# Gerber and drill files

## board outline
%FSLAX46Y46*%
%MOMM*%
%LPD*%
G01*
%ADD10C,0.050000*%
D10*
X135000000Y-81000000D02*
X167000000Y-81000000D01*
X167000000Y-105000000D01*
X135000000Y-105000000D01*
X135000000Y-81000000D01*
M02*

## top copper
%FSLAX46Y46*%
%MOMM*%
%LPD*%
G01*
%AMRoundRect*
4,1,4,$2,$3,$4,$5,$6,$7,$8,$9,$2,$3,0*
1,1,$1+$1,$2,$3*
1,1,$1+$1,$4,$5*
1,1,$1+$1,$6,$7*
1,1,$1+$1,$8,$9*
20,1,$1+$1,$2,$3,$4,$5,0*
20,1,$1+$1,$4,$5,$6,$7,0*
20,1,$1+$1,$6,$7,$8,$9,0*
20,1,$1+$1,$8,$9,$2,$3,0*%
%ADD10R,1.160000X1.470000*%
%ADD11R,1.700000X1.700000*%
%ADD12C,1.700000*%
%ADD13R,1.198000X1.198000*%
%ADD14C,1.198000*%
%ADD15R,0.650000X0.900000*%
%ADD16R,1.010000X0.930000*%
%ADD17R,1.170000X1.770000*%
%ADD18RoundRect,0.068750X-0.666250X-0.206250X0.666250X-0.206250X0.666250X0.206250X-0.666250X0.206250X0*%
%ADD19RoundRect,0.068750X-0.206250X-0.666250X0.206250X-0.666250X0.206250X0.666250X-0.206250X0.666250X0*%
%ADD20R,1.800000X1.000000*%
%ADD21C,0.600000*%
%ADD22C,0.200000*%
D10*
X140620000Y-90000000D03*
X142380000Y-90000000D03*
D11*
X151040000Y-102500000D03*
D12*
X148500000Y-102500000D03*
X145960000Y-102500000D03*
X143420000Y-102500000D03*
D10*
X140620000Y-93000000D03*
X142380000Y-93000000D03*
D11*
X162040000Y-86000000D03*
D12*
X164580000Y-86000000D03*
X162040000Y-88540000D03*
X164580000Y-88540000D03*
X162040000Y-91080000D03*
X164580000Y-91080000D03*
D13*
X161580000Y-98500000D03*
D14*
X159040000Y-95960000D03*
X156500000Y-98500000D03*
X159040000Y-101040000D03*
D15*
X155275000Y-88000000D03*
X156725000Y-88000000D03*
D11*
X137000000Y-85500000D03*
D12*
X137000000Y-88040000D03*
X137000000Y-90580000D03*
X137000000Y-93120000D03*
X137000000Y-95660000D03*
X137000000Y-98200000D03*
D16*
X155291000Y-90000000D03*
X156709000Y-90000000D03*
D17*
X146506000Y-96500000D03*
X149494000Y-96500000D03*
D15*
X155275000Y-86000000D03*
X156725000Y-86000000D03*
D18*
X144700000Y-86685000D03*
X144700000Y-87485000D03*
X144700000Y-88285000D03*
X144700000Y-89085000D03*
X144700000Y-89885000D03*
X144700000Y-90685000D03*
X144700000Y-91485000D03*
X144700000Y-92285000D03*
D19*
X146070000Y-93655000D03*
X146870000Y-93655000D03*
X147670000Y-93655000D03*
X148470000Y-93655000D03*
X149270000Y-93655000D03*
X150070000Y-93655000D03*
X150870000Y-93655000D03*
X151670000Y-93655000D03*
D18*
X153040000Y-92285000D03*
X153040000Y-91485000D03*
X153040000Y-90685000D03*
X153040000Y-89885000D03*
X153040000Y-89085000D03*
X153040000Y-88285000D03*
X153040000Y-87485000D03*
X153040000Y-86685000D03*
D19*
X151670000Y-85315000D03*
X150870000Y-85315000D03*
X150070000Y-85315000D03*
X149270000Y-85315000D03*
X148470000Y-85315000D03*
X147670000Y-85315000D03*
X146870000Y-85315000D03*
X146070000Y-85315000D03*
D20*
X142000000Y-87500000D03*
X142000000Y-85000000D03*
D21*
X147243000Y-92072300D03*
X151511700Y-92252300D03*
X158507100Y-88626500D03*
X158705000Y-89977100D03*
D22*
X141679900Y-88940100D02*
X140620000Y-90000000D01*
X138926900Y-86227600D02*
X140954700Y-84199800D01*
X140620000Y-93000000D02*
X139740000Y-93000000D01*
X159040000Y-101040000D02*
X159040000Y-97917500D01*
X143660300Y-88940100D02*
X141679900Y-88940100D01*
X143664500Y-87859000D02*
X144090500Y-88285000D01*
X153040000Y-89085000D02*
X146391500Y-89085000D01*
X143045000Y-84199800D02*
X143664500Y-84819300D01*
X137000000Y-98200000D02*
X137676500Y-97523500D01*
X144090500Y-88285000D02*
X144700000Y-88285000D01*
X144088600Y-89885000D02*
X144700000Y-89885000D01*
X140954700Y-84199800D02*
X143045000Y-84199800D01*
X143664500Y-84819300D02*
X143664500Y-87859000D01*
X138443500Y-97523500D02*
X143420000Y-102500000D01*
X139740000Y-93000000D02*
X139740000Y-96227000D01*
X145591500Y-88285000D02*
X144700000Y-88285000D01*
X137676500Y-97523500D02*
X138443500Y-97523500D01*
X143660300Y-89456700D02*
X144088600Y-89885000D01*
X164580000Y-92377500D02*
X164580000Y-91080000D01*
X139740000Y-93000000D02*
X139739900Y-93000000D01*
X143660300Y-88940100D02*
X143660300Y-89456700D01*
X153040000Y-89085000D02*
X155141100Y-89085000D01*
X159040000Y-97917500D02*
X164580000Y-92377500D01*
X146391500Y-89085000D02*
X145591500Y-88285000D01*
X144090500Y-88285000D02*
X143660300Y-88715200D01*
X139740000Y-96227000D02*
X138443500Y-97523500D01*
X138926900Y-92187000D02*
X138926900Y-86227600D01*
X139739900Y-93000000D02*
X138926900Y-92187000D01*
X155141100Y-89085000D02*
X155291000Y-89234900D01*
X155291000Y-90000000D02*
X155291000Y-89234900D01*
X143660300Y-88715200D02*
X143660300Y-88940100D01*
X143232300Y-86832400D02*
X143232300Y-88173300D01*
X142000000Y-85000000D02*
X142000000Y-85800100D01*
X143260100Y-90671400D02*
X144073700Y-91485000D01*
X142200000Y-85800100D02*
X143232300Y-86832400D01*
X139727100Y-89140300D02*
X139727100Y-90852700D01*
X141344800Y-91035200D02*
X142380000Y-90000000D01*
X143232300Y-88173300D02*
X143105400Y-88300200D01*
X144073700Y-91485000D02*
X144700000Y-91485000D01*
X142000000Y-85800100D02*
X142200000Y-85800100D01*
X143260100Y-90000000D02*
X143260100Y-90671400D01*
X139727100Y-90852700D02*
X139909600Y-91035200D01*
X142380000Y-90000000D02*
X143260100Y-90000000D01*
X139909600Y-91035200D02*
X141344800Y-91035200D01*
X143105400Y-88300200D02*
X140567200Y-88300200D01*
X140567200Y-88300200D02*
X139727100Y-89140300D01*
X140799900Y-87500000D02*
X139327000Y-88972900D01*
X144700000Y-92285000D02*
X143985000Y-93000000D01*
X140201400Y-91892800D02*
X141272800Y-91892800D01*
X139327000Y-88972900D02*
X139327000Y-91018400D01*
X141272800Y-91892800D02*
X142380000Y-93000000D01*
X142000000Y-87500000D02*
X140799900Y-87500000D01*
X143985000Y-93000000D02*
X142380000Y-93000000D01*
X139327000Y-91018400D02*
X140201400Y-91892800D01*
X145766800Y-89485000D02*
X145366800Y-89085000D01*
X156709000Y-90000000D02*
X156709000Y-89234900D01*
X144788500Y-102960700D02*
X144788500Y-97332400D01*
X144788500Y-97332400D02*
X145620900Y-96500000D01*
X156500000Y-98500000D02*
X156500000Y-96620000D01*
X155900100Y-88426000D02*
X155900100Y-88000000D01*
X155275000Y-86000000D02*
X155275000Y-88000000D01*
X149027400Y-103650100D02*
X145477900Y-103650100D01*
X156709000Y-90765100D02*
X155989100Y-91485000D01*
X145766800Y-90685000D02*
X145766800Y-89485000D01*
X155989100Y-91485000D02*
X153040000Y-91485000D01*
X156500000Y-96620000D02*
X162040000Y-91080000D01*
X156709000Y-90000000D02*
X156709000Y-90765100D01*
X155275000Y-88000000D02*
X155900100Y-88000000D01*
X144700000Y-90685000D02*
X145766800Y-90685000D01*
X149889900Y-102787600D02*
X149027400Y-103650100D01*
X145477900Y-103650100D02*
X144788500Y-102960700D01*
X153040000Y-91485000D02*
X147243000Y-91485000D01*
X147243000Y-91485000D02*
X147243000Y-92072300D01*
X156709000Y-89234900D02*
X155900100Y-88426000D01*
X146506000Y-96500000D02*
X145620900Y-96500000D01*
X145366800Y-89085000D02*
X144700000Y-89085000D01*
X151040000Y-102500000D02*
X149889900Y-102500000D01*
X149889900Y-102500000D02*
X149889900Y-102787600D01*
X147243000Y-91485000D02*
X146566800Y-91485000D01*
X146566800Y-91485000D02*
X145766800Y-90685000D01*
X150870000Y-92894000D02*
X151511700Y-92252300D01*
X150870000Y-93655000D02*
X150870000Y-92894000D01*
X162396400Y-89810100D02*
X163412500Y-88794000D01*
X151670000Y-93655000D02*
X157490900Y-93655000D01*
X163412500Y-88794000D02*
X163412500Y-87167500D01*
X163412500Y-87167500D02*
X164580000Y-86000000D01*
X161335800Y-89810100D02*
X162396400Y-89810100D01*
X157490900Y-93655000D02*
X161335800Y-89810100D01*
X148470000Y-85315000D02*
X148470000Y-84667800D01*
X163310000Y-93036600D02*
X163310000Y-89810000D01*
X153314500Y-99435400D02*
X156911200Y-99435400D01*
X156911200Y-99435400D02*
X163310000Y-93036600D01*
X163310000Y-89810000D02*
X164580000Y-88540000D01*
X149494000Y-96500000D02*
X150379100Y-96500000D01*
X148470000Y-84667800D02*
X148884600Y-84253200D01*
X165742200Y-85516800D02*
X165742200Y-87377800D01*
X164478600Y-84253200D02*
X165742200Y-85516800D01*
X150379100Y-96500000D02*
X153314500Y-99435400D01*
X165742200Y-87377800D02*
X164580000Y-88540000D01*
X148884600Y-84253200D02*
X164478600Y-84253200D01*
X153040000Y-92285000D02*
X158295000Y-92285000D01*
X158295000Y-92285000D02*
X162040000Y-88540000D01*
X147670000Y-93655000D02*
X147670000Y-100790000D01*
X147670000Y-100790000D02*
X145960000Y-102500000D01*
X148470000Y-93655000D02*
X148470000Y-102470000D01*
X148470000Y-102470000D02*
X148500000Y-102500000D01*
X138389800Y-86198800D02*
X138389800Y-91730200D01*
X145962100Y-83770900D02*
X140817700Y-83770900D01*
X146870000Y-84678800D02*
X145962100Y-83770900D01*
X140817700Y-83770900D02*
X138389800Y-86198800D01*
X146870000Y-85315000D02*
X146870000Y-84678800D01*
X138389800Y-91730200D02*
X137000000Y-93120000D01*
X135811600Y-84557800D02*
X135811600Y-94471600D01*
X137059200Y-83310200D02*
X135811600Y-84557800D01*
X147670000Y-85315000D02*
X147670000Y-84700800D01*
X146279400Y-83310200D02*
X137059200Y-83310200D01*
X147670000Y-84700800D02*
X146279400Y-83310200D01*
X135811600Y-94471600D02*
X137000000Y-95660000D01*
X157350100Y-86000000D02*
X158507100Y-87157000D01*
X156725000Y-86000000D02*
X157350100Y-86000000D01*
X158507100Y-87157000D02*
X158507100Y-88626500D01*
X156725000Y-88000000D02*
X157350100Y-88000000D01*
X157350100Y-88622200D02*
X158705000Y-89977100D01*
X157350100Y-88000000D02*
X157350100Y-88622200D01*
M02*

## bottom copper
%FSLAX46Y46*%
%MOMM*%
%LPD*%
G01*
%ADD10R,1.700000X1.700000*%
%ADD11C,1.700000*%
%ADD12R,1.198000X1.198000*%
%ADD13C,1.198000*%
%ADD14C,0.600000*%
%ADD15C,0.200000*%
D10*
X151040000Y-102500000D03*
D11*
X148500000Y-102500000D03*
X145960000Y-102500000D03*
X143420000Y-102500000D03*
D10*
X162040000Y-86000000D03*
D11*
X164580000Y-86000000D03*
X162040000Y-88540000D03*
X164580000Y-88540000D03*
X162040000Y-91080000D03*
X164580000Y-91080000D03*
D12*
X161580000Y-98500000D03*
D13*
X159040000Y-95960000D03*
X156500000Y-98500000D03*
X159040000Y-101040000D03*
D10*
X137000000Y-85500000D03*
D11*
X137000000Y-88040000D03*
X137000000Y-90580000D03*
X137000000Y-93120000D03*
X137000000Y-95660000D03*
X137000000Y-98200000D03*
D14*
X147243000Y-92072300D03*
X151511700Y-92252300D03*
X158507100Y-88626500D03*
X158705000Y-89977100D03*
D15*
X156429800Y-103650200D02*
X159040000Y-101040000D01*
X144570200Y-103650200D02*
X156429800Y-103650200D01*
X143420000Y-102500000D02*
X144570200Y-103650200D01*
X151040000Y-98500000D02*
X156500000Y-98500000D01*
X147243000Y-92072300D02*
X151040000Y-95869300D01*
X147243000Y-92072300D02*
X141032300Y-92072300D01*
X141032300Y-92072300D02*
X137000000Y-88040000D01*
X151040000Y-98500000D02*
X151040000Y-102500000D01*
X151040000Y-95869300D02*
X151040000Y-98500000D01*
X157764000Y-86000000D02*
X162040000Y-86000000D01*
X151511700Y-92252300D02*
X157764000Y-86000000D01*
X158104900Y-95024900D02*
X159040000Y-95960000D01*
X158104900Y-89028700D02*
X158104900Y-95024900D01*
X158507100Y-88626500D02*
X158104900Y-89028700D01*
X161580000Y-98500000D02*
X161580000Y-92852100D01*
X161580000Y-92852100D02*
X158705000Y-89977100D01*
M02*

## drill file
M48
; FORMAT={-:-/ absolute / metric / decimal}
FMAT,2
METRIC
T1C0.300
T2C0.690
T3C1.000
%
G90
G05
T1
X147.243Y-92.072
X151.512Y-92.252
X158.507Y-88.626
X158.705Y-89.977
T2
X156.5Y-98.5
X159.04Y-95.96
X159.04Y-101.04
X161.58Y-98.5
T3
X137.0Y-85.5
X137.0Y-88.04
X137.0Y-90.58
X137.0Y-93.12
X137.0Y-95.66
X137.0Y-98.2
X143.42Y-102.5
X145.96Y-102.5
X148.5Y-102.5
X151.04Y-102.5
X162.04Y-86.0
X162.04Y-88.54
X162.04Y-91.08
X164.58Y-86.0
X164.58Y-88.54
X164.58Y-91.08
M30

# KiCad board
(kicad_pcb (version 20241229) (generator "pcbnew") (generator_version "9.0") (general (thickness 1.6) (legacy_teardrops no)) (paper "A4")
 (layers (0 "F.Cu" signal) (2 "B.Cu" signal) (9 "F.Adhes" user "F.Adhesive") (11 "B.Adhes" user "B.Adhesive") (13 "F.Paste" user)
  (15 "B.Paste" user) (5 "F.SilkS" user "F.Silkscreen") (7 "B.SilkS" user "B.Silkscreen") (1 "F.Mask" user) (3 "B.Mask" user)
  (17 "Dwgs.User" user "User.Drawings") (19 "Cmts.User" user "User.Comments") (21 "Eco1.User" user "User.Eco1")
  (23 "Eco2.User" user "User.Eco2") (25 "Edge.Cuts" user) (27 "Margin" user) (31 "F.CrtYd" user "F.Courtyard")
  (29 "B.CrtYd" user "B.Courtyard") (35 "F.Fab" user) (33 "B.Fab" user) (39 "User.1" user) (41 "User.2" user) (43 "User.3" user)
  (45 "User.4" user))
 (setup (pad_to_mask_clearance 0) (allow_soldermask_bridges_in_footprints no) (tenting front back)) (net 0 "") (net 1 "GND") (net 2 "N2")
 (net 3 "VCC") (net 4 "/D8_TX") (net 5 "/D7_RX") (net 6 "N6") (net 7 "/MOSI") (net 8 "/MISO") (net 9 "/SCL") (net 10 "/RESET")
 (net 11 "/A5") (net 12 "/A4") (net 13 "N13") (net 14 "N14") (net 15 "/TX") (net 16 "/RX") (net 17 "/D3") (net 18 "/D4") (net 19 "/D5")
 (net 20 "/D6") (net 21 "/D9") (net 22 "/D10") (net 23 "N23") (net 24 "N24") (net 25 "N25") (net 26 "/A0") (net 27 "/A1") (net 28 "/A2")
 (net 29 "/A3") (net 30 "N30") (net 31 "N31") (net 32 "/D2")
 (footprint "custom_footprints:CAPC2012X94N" (layer "F.Cu") (at 141.5 90)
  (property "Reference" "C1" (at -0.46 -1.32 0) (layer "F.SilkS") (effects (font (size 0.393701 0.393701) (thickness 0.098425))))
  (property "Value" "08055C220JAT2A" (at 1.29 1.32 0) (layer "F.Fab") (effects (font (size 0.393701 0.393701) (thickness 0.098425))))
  (pad "1" smd rect (at -0.88 0) (size 1.16 1.47) (layers "F.Cu" "F.Mask" "F.Paste") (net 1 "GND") (solder_mask_margin 0.102))
  (pad "2" smd rect (at 0.88 0) (size 1.16 1.47) (layers "F.Cu" "F.Mask" "F.Paste") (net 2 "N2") (solder_mask_margin 0.102)))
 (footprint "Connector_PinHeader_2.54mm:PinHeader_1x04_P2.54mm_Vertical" (layer "F.Cu") (at 151.04 102.5 -90)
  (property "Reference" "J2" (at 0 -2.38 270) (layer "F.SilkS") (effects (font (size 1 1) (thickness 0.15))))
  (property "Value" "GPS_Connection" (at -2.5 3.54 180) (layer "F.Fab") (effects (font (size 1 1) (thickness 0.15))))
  (pad "1" thru_hole rect (at 0 0 270) (size 1.7 1.7) (drill 1) (layers "*.Cu" "*.Mask") (remove_unused_layers no) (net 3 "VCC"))
  (pad "2" thru_hole circle (at 0 2.54 270) (size 1.7 1.7) (drill 1) (layers "*.Cu" "*.Mask") (remove_unused_layers no) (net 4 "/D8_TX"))
  (pad "3" thru_hole circle (at 0 5.08 270) (size 1.7 1.7) (drill 1) (layers "*.Cu" "*.Mask") (remove_unused_layers no) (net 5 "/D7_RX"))
  (pad "4" thru_hole circle (at 0 7.62 270) (size 1.7 1.7) (drill 1) (layers "*.Cu" "*.Mask") (remove_unused_layers no) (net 1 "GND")))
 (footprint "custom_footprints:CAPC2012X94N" (layer "F.Cu") (at 141.5 93)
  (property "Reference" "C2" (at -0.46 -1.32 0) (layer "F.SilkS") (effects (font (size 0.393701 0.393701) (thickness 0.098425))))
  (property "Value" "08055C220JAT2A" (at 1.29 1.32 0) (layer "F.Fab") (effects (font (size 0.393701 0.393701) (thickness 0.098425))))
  (pad "1" smd rect (at -0.88 0) (size 1.16 1.47) (layers "F.Cu" "F.Mask" "F.Paste") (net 1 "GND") (solder_mask_margin 0.102))
  (pad "2" smd rect (at 0.88 0) (size 1.16 1.47) (layers "F.Cu" "F.Mask" "F.Paste") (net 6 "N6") (solder_mask_margin 0.102)))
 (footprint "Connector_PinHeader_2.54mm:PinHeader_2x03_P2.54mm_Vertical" (layer "F.Cu") (at 162.04 86)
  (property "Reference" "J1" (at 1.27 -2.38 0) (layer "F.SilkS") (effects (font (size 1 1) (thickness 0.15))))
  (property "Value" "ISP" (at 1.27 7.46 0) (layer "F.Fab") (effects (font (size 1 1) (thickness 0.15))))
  (pad "1" thru_hole rect (at 0 0) (size 1.7 1.7) (drill 1) (layers "*.Cu" "*.Mask") (remove_unused_layers no) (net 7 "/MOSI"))
  (pad "2" thru_hole circle (at 2.54 0) (size 1.7 1.7) (drill 1) (layers "*.Cu" "*.Mask") (remove_unused_layers no) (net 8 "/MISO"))
  (pad "3" thru_hole circle (at 0 2.54) (size 1.7 1.7) (drill 1) (layers "*.Cu" "*.Mask") (remove_unused_layers no) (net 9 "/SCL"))
  (pad "4" thru_hole circle (at 2.54 2.54) (size 1.7 1.7) (drill 1) (layers "*.Cu" "*.Mask") (remove_unused_layers no) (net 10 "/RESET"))
  (pad "5" thru_hole circle (at 0 5.08) (size 1.7 1.7) (drill 1) (layers "*.Cu" "*.Mask") (remove_unused_layers no) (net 3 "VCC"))
  (pad "6" thru_hole circle (at 2.54 5.08) (size 1.7 1.7) (drill 1) (layers "*.Cu" "*.Mask") (remove_unused_layers no) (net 1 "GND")))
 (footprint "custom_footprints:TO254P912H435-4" (layer "F.Cu") (at 159.04 98.5 180)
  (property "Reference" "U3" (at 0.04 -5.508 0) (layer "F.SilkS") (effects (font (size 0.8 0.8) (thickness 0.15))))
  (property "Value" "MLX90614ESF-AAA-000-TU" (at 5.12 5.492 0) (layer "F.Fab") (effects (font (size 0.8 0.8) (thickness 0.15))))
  (pad "1" thru_hole rect (at -2.54 0 180) (size 1.198 1.198) (drill 0.69) (layers "*.Cu" "*.Mask") (remove_unused_layers no) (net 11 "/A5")
   (solder_mask_margin 0.102))
  (pad "2" thru_hole circle (at 0 2.54 180) (size 1.198 1.198) (drill 0.69) (layers "*.Cu" "*.Mask") (remove_unused_layers no)
   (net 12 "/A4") (solder_mask_margin 0.102))
  (pad "3" thru_hole circle (at 2.54 0 180) (size 1.198 1.198) (drill 0.69) (layers "*.Cu" "*.Mask") (remove_unused_layers no) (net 3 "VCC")
   (solder_mask_margin 0.102))
  (pad "4" thru_hole circle (at 0 -2.54 180) (size 1.198 1.198) (drill 0.69) (layers "*.Cu" "*.Mask") (remove_unused_layers no)
   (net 1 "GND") (solder_mask_margin 0.102)))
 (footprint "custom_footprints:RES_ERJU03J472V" (layer "F.Cu") (at 156 88)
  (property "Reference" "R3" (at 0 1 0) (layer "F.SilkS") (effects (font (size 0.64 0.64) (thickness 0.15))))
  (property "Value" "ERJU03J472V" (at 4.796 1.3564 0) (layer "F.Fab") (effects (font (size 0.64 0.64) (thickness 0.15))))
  (pad "1" smd rect (at -0.725 0) (size 0.65 0.9) (layers "F.Cu" "F.Mask" "F.Paste") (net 3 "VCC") (solder_mask_margin 0.102))
  (pad "2" smd rect (at 0.725 0) (size 0.65 0.9) (layers "F.Cu" "F.Mask" "F.Paste") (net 11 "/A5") (solder_mask_margin 0.102)))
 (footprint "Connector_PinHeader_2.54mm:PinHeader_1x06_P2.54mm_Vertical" (layer "F.Cu") (at 137 85.5)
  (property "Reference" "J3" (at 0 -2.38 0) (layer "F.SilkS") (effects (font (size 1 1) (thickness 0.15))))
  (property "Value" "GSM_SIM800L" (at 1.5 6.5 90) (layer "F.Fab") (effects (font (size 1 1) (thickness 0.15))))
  (pad "1" thru_hole rect (at 0 0) (size 1.7 1.7) (drill 1) (layers "*.Cu" "*.Mask") (remove_unused_layers no) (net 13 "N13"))
  (pad "2" thru_hole circle (at 0 2.54) (size 1.7 1.7) (drill 1) (layers "*.Cu" "*.Mask") (remove_unused_layers no) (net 3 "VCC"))
  (pad "3" thru_hole circle (at 0 5.08) (size 1.7 1.7) (drill 1) (layers "*.Cu" "*.Mask") (remove_unused_layers no) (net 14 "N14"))
  (pad "4" thru_hole circle (at 0 7.62) (size 1.7 1.7) (drill 1) (layers "*.Cu" "*.Mask") (remove_unused_layers no) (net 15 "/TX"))
  (pad "5" thru_hole circle (at 0 10.16) (size 1.7 1.7) (drill 1) (layers "*.Cu" "*.Mask") (remove_unused_layers no) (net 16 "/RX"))
  (pad "6" thru_hole circle (at 0 12.7) (size 1.7 1.7) (drill 1) (layers "*.Cu" "*.Mask") (remove_unused_layers no) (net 1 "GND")))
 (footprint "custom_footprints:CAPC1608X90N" (layer "F.Cu") (at 156 90)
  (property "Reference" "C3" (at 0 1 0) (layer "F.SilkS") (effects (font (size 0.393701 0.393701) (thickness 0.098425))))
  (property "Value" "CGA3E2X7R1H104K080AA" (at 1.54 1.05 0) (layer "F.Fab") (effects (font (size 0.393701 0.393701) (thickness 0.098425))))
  (pad "1" smd rect (at -0.709 0) (size 1.01 0.93) (layers "F.Cu" "F.Mask" "F.Paste") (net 1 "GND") (solder_mask_margin 0.102))
  (pad "2" smd rect (at 0.709 0) (size 1.01 0.93) (layers "F.Cu" "F.Mask" "F.Paste") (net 3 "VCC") (solder_mask_margin 0.102)))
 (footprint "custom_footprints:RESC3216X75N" (layer "F.Cu") (at 148 96.5)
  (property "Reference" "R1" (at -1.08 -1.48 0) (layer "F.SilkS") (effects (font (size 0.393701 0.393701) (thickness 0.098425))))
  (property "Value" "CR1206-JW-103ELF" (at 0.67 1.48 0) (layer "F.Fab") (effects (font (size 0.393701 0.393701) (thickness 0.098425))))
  (pad "1" smd rect (at -1.494 0) (size 1.17 1.77) (layers "F.Cu" "F.Mask" "F.Paste") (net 3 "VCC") (solder_mask_margin 0.102))
  (pad "2" smd rect (at 1.494 0) (size 1.17 1.77) (layers "F.Cu" "F.Mask" "F.Paste") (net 10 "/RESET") (solder_mask_margin 0.102)))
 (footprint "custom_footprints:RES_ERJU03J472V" (layer "F.Cu") (at 156 86)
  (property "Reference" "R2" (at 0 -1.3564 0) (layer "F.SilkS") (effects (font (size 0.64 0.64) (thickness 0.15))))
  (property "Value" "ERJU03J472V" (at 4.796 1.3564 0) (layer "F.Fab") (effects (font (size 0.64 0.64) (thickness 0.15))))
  (pad "1" smd rect (at -0.725 0) (size 0.65 0.9) (layers "F.Cu" "F.Mask" "F.Paste") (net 3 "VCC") (solder_mask_margin 0.102))
  (pad "2" smd rect (at 0.725 0) (size 0.65 0.9) (layers "F.Cu" "F.Mask" "F.Paste") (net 12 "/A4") (solder_mask_margin 0.102)))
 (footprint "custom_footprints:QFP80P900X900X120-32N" (layer "F.Cu") (at 148.87 89.485)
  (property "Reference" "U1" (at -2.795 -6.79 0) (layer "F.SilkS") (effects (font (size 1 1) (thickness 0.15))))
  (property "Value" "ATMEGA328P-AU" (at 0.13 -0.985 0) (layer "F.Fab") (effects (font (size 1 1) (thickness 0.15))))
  (pad "1" smd roundrect (at -4.17 -2.8) (size 1.47 0.55) (layers "F.Cu" "F.Mask" "F.Paste") (roundrect_rratio 0.125) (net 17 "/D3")
   (solder_mask_margin 0.102))
  (pad "2" smd roundrect (at -4.17 -2) (size 1.47 0.55) (layers "F.Cu" "F.Mask" "F.Paste") (roundrect_rratio 0.125) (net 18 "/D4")
   (solder_mask_margin 0.102))
  (pad "3" smd roundrect (at -4.17 -1.2) (size 1.47 0.55) (layers "F.Cu" "F.Mask" "F.Paste") (roundrect_rratio 0.125) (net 1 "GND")
   (solder_mask_margin 0.102))
  (pad "4" smd roundrect (at -4.17 -0.4) (size 1.47 0.55) (layers "F.Cu" "F.Mask" "F.Paste") (roundrect_rratio 0.125) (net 3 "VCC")
   (solder_mask_margin 0.102))
  (pad "5" smd roundrect (at -4.17 0.4) (size 1.47 0.55) (layers "F.Cu" "F.Mask" "F.Paste") (roundrect_rratio 0.125) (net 1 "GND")
   (solder_mask_margin 0.102))
  (pad "6" smd roundrect (at -4.17 1.2) (size 1.47 0.55) (layers "F.Cu" "F.Mask" "F.Paste") (roundrect_rratio 0.125) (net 3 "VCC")
   (solder_mask_margin 0.102))
  (pad "7" smd roundrect (at -4.17 2) (size 1.47 0.55) (layers "F.Cu" "F.Mask" "F.Paste") (roundrect_rratio 0.125) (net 2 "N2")
   (solder_mask_margin 0.102))
  (pad "8" smd roundrect (at -4.17 2.8) (size 1.47 0.55) (layers "F.Cu" "F.Mask" "F.Paste") (roundrect_rratio 0.125) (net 6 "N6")
   (solder_mask_margin 0.102))
  (pad "9" smd roundrect (at -2.8 4.17) (size 0.55 1.47) (layers "F.Cu" "F.Mask" "F.Paste") (roundrect_rratio 0.125) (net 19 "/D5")
   (solder_mask_margin 0.102))
  (pad "10" smd roundrect (at -2 4.17) (size 0.55 1.47) (layers "F.Cu" "F.Mask" "F.Paste") (roundrect_rratio 0.125) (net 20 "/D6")
   (solder_mask_margin 0.102))
  (pad "11" smd roundrect (at -1.2 4.17) (size 0.55 1.47) (layers "F.Cu" "F.Mask" "F.Paste") (roundrect_rratio 0.125) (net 5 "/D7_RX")
   (solder_mask_margin 0.102))
  (pad "12" smd roundrect (at -0.4 4.17) (size 0.55 1.47) (layers "F.Cu" "F.Mask" "F.Paste") (roundrect_rratio 0.125) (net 4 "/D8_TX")
   (solder_mask_margin 0.102))
  (pad "13" smd roundrect (at 0.4 4.17) (size 0.55 1.47) (layers "F.Cu" "F.Mask" "F.Paste") (roundrect_rratio 0.125) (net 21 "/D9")
   (solder_mask_margin 0.102))
  (pad "14" smd roundrect (at 1.2 4.17) (size 0.55 1.47) (layers "F.Cu" "F.Mask" "F.Paste") (roundrect_rratio 0.125) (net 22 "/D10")
   (solder_mask_margin 0.102))
  (pad "15" smd roundrect (at 2 4.17) (size 0.55 1.47) (layers "F.Cu" "F.Mask" "F.Paste") (roundrect_rratio 0.125) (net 7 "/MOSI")
   (solder_mask_margin 0.102))
  (pad "16" smd roundrect (at 2.8 4.17) (size 0.55 1.47) (layers "F.Cu" "F.Mask" "F.Paste") (roundrect_rratio 0.125) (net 8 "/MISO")
   (solder_mask_margin 0.102))
  (pad "17" smd roundrect (at 4.17 2.8) (size 1.47 0.55) (layers "F.Cu" "F.Mask" "F.Paste") (roundrect_rratio 0.125) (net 9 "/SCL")
   (solder_mask_margin 0.102))
  (pad "18" smd roundrect (at 4.17 2) (size 1.47 0.55) (layers "F.Cu" "F.Mask" "F.Paste") (roundrect_rratio 0.125) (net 3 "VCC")
   (solder_mask_margin 0.102))
  (pad "19" smd roundrect (at 4.17 1.2) (size 1.47 0.55) (layers "F.Cu" "F.Mask" "F.Paste") (roundrect_rratio 0.125) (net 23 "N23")
   (solder_mask_margin 0.102))
  (pad "20" smd roundrect (at 4.17 0.4) (size 1.47 0.55) (layers "F.Cu" "F.Mask" "F.Paste") (roundrect_rratio 0.125) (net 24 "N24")
   (solder_mask_margin 0.102))
  (pad "21" smd roundrect (at 4.17 -0.4) (size 1.47 0.55) (layers "F.Cu" "F.Mask" "F.Paste") (roundrect_rratio 0.125) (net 1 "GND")
   (solder_mask_margin 0.102))
  (pad "22" smd roundrect (at 4.17 -1.2) (size 1.47 0.55) (layers "F.Cu" "F.Mask" "F.Paste") (roundrect_rratio 0.125) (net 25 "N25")
   (solder_mask_margin 0.102))
  (pad "23" smd roundrect (at 4.17 -2) (size 1.47 0.55) (layers "F.Cu" "F.Mask" "F.Paste") (roundrect_rratio 0.125) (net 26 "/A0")
   (solder_mask_margin 0.102))
  (pad "24" smd roundrect (at 4.17 -2.8) (size 1.47 0.55) (layers "F.Cu" "F.Mask" "F.Paste") (roundrect_rratio 0.125) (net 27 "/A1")
   (solder_mask_margin 0.102))
  (pad "25" smd roundrect (at 2.8 -4.17) (size 0.55 1.47) (layers "F.Cu" "F.Mask" "F.Paste") (roundrect_rratio 0.125) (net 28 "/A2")
   (solder_mask_margin 0.102))
  (pad "26" smd roundrect (at 2 -4.17) (size 0.55 1.47) (layers "F.Cu" "F.Mask" "F.Paste") (roundrect_rratio 0.125) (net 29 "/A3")
   (solder_mask_margin 0.102))
  (pad "27" smd roundrect (at 1.2 -4.17) (size 0.55 1.47) (layers "F.Cu" "F.Mask" "F.Paste") (roundrect_rratio 0.125) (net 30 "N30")
   (solder_mask_margin 0.102))
  (pad "28" smd roundrect (at 0.4 -4.17) (size 0.55 1.47) (layers "F.Cu" "F.Mask" "F.Paste") (roundrect_rratio 0.125) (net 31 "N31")
   (solder_mask_margin 0.102))
  (pad "29" smd roundrect (at -0.4 -4.17) (size 0.55 1.47) (layers "F.Cu" "F.Mask" "F.Paste") (roundrect_rratio 0.125) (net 10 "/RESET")
   (solder_mask_margin 0.102))
  (pad "30" smd roundrect (at -1.2 -4.17) (size 0.55 1.47) (layers "F.Cu" "F.Mask" "F.Paste") (roundrect_rratio 0.125) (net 16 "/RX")
   (solder_mask_margin 0.102))
  (pad "31" smd roundrect (at -2 -4.17) (size 0.55 1.47) (layers "F.Cu" "F.Mask" "F.Paste") (roundrect_rratio 0.125) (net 15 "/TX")
   (solder_mask_margin 0.102))
  (pad "32" smd roundrect (at -2.8 -4.17) (size 0.55 1.47) (layers "F.Cu" "F.Mask" "F.Paste") (roundrect_rratio 0.125) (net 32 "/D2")
   (solder_mask_margin 0.102)))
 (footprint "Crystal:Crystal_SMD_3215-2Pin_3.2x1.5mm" (layer "F.Cu") (at 142 86.25 -90)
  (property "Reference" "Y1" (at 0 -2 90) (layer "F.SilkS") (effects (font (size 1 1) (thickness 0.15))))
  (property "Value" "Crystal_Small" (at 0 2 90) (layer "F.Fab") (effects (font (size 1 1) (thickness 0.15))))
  (pad "1" smd rect (at 1.25 0 270) (size 1 1.8) (layers "F.Cu" "F.Mask" "F.Paste") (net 6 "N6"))
  (pad "2" smd rect (at -1.25 0 270) (size 1 1.8) (layers "F.Cu" "F.Mask" "F.Paste") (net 2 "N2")))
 (gr_rect (start 135 81) (end 167 105) (stroke (width 0.05) (type default)) (fill no) (layer "Edge.Cuts"))
 (segment (start 141.6799 88.9401) (end 140.62 90) (width 0.2) (layer "F.Cu") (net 1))
 (segment (start 138.9269 86.2276) (end 140.9547 84.1998) (width 0.2) (layer "F.Cu") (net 1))
 (segment (start 140.62 93) (end 139.74 93) (width 0.2) (layer "F.Cu") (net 1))
 (segment (start 159.04 101.04) (end 159.04 97.9175) (width 0.2) (layer "F.Cu") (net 1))
 (segment (start 143.6603 88.9401) (end 141.6799 88.9401) (width 0.2) (layer "F.Cu") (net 1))
 (segment (start 143.6645 87.859) (end 144.0905 88.285) (width 0.2) (layer "F.Cu") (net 1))
 (segment (start 153.04 89.085) (end 146.3915 89.085) (width 0.2) (layer "F.Cu") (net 1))
 (segment (start 143.045 84.1998) (end 143.6645 84.8193) (width 0.2) (layer "F.Cu") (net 1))
 (segment (start 137 98.2) (end 137.6765 97.5235) (width 0.2) (layer "F.Cu") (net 1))
 (segment (start 144.0905 88.285) (end 144.7 88.285) (width 0.2) (layer "F.Cu") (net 1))
 (segment (start 144.0886 89.885) (end 144.7 89.885) (width 0.2) (layer "F.Cu") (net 1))
 (segment (start 140.9547 84.1998) (end 143.045 84.1998) (width 0.2) (layer "F.Cu") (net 1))
 (segment (start 143.6645 84.8193) (end 143.6645 87.859) (width 0.2) (layer "F.Cu") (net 1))
 (segment (start 138.4435 97.5235) (end 143.42 102.5) (width 0.2) (layer "F.Cu") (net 1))
 (segment (start 139.74 93) (end 139.74 96.227) (width 0.2) (layer "F.Cu") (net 1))
 (segment (start 145.5915 88.285) (end 144.7 88.285) (width 0.2) (layer "F.Cu") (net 1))
 (segment (start 137.6765 97.5235) (end 138.4435 97.5235) (width 0.2) (layer "F.Cu") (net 1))
 (segment (start 143.6603 89.4567) (end 144.0886 89.885) (width 0.2) (layer "F.Cu") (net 1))
 (segment (start 164.58 92.3775) (end 164.58 91.08) (width 0.2) (layer "F.Cu") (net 1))
 (segment (start 139.74 93) (end 139.7399 93) (width 0.2) (layer "F.Cu") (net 1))
 (segment (start 143.6603 88.9401) (end 143.6603 89.4567) (width 0.2) (layer "F.Cu") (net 1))
 (segment (start 153.04 89.085) (end 155.1411 89.085) (width 0.2) (layer "F.Cu") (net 1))
 (segment (start 159.04 97.9175) (end 164.58 92.3775) (width 0.2) (layer "F.Cu") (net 1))
 (segment (start 146.3915 89.085) (end 145.5915 88.285) (width 0.2) (layer "F.Cu") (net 1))
 (segment (start 144.0905 88.285) (end 143.6603 88.7152) (width 0.2) (layer "F.Cu") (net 1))
 (segment (start 139.74 96.227) (end 138.4435 97.5235) (width 0.2) (layer "F.Cu") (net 1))
 (segment (start 138.9269 92.187) (end 138.9269 86.2276) (width 0.2) (layer "F.Cu") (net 1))
 (segment (start 139.7399 93) (end 138.9269 92.187) (width 0.2) (layer "F.Cu") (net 1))
 (segment (start 155.1411 89.085) (end 155.291 89.2349) (width 0.2) (layer "F.Cu") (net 1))
 (segment (start 155.291 90) (end 155.291 89.2349) (width 0.2) (layer "F.Cu") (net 1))
 (segment (start 143.6603 88.7152) (end 143.6603 88.9401) (width 0.2) (layer "F.Cu") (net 1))
 (segment (start 156.4298 103.6502) (end 159.04 101.04) (width 0.2) (layer "B.Cu") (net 1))
 (segment (start 144.5702 103.6502) (end 156.4298 103.6502) (width 0.2) (layer "B.Cu") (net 1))
 (segment (start 143.42 102.5) (end 144.5702 103.6502) (width 0.2) (layer "B.Cu") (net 1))
 (segment (start 143.2323 86.8324) (end 143.2323 88.1733) (width 0.2) (layer "F.Cu") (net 2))
 (segment (start 142 85) (end 142 85.8001) (width 0.2) (layer "F.Cu") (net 2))
 (segment (start 143.2601 90.6714) (end 144.0737 91.485) (width 0.2) (layer "F.Cu") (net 2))
 (segment (start 142.2 85.8001) (end 143.2323 86.8324) (width 0.2) (layer "F.Cu") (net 2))
 (segment (start 139.7271 89.1403) (end 139.7271 90.8527) (width 0.2) (layer "F.Cu") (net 2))
 (segment (start 141.3448 91.0352) (end 142.38 90) (width 0.2) (layer "F.Cu") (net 2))
 (segment (start 143.2323 88.1733) (end 143.1054 88.3002) (width 0.2) (layer "F.Cu") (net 2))
 (segment (start 144.0737 91.485) (end 144.7 91.485) (width 0.2) (layer "F.Cu") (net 2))
 (segment (start 142 85.8001) (end 142.2 85.8001) (width 0.2) (layer "F.Cu") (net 2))
 (segment (start 143.2601 90) (end 143.2601 90.6714) (width 0.2) (layer "F.Cu") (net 2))
 (segment (start 139.7271 90.8527) (end 139.9096 91.0352) (width 0.2) (layer "F.Cu") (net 2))
 (segment (start 142.38 90) (end 143.2601 90) (width 0.2) (layer "F.Cu") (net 2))
 (segment (start 139.9096 91.0352) (end 141.3448 91.0352) (width 0.2) (layer "F.Cu") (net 2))
 (segment (start 143.1054 88.3002) (end 140.5672 88.3002) (width 0.2) (layer "F.Cu") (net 2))
 (segment (start 140.5672 88.3002) (end 139.7271 89.1403) (width 0.2) (layer "F.Cu") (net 2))
 (segment (start 140.7999 87.5) (end 139.327 88.9729) (width 0.2) (layer "F.Cu") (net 6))
 (segment (start 144.7 92.285) (end 143.985 93) (width 0.2) (layer "F.Cu") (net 6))
 (segment (start 140.2014 91.8928) (end 141.2728 91.8928) (width 0.2) (layer "F.Cu") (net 6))
 (segment (start 139.327 88.9729) (end 139.327 91.0184) (width 0.2) (layer "F.Cu") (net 6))
 (segment (start 141.2728 91.8928) (end 142.38 93) (width 0.2) (layer "F.Cu") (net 6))
 (segment (start 142 87.5) (end 140.7999 87.5) (width 0.2) (layer "F.Cu") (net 6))
 (segment (start 143.985 93) (end 142.38 93) (width 0.2) (layer "F.Cu") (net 6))
 (segment (start 139.327 91.0184) (end 140.2014 91.8928) (width 0.2) (layer "F.Cu") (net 6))
 (segment (start 145.7668 89.485) (end 145.3668 89.085) (width 0.2) (layer "F.Cu") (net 3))
 (segment (start 156.709 90) (end 156.709 89.2349) (width 0.2) (layer "F.Cu") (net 3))
 (segment (start 144.7885 102.9607) (end 144.7885 97.3324) (width 0.2) (layer "F.Cu") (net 3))
 (segment (start 144.7885 97.3324) (end 145.6209 96.5) (width 0.2) (layer "F.Cu") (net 3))
 (segment (start 156.5 98.5) (end 156.5 96.62) (width 0.2) (layer "F.Cu") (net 3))
 (segment (start 155.9001 88.426) (end 155.9001 88) (width 0.2) (layer "F.Cu") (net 3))
 (segment (start 155.275 86) (end 155.275 88) (width 0.2) (layer "F.Cu") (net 3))
 (segment (start 149.0274 103.6501) (end 145.4779 103.6501) (width 0.2) (layer "F.Cu") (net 3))
 (segment (start 156.709 90.7651) (end 155.9891 91.485) (width 0.2) (layer "F.Cu") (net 3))
 (segment (start 145.7668 90.685) (end 145.7668 89.485) (width 0.2) (layer "F.Cu") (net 3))
 (segment (start 155.9891 91.485) (end 153.04 91.485) (width 0.2) (layer "F.Cu") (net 3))
 (segment (start 156.5 96.62) (end 162.04 91.08) (width 0.2) (layer "F.Cu") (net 3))
 (segment (start 156.709 90) (end 156.709 90.7651) (width 0.2) (layer "F.Cu") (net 3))
 (segment (start 155.275 88) (end 155.9001 88) (width 0.2) (layer "F.Cu") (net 3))
 (segment (start 144.7 90.685) (end 145.7668 90.685) (width 0.2) (layer "F.Cu") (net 3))
 (segment (start 149.8899 102.7876) (end 149.0274 103.6501) (width 0.2) (layer "F.Cu") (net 3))
 (segment (start 145.4779 103.6501) (end 144.7885 102.9607) (width 0.2) (layer "F.Cu") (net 3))
 (segment (start 153.04 91.485) (end 147.243 91.485) (width 0.2) (layer "F.Cu") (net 3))
 (segment (start 147.243 91.485) (end 147.243 92.0723) (width 0.2) (layer "F.Cu") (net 3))
 (segment (start 156.709 89.2349) (end 155.9001 88.426) (width 0.2) (layer "F.Cu") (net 3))
 (segment (start 146.506 96.5) (end 145.6209 96.5) (width 0.2) (layer "F.Cu") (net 3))
 (segment (start 145.3668 89.085) (end 144.7 89.085) (width 0.2) (layer "F.Cu") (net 3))
 (segment (start 151.04 102.5) (end 149.8899 102.5) (width 0.2) (layer "F.Cu") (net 3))
 (segment (start 149.8899 102.5) (end 149.8899 102.7876) (width 0.2) (layer "F.Cu") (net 3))
 (segment (start 147.243 91.485) (end 146.5668 91.485) (width 0.2) (layer "F.Cu") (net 3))
 (segment (start 146.5668 91.485) (end 145.7668 90.685) (width 0.2) (layer "F.Cu") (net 3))
 (via (at 147.243 92.0723) (size 0.6) (drill 0.3) (layers "F.Cu" "B.Cu") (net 3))
 (segment (start 151.04 98.5) (end 156.5 98.5) (width 0.2) (layer "B.Cu") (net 3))
 (segment (start 147.243 92.0723) (end 151.04 95.8693) (width 0.2) (layer "B.Cu") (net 3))
 (segment (start 147.243 92.0723) (end 141.0323 92.0723) (width 0.2) (layer "B.Cu") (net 3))
 (segment (start 141.0323 92.0723) (end 137 88.04) (width 0.2) (layer "B.Cu") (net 3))
 (segment (start 151.04 98.5) (end 151.04 102.5) (width 0.2) (layer "B.Cu") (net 3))
 (segment (start 151.04 95.8693) (end 151.04 98.5) (width 0.2) (layer "B.Cu") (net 3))
 (segment (start 150.87 92.894) (end 151.5117 92.2523) (width 0.2) (layer "F.Cu") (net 7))
 (segment (start 150.87 93.655) (end 150.87 92.894) (width 0.2) (layer "F.Cu") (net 7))
 (via (at 151.5117 92.2523) (size 0.6) (drill 0.3) (layers "F.Cu" "B.Cu") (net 7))
 (segment (start 157.764 86) (end 162.04 86) (width 0.2) (layer "B.Cu") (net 7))
 (segment (start 151.5117 92.2523) (end 157.764 86) (width 0.2) (layer "B.Cu") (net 7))
 (segment (start 162.3964 89.8101) (end 163.4125 88.794) (width 0.2) (layer "F.Cu") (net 8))
 (segment (start 151.67 93.655) (end 157.4909 93.655) (width 0.2) (layer "F.Cu") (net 8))
 (segment (start 163.4125 88.794) (end 163.4125 87.1675) (width 0.2) (layer "F.Cu") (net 8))
 (segment (start 163.4125 87.1675) (end 164.58 86) (width 0.2) (layer "F.Cu") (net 8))
 (segment (start 161.3358 89.8101) (end 162.3964 89.8101) (width 0.2) (layer "F.Cu") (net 8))
 (segment (start 157.4909 93.655) (end 161.3358 89.8101) (width 0.2) (layer "F.Cu") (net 8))
 (segment (start 148.47 85.315) (end 148.47 84.6678) (width 0.2) (layer "F.Cu") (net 10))
 (segment (start 163.31 93.0366) (end 163.31 89.81) (width 0.2) (layer "F.Cu") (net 10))
 (segment (start 153.3145 99.4354) (end 156.9112 99.4354) (width 0.2) (layer "F.Cu") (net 10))
 (segment (start 156.9112 99.4354) (end 163.31 93.0366) (width 0.2) (layer "F.Cu") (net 10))
 (segment (start 163.31 89.81) (end 164.58 88.54) (width 0.2) (layer "F.Cu") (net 10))
 (segment (start 149.494 96.5) (end 150.3791 96.5) (width 0.2) (layer "F.Cu") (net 10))
 (segment (start 148.47 84.6678) (end 148.8846 84.2532) (width 0.2) (layer "F.Cu") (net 10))
 (segment (start 165.7422 85.5168) (end 165.7422 87.3778) (width 0.2) (layer "F.Cu") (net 10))
 (segment (start 164.4786 84.2532) (end 165.7422 85.5168) (width 0.2) (layer "F.Cu") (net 10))
 (segment (start 150.3791 96.5) (end 153.3145 99.4354) (width 0.2) (layer "F.Cu") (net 10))
 (segment (start 165.7422 87.3778) (end 164.58 88.54) (width 0.2) (layer "F.Cu") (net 10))
 (segment (start 148.8846 84.2532) (end 164.4786 84.2532) (width 0.2) (layer "F.Cu") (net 10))
 (segment (start 153.04 92.285) (end 158.295 92.285) (width 0.2) (layer "F.Cu") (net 9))
 (segment (start 158.295 92.285) (end 162.04 88.54) (width 0.2) (layer "F.Cu") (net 9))
 (segment (start 147.67 93.655) (end 147.67 100.79) (width 0.2) (layer "F.Cu") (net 5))
 (segment (start 147.67 100.79) (end 145.96 102.5) (width 0.2) (layer "F.Cu") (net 5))
 (segment (start 148.47 93.655) (end 148.47 102.47) (width 0.2) (layer "F.Cu") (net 4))
 (segment (start 148.47 102.47) (end 148.5 102.5) (width 0.2) (layer "F.Cu") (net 4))
 (segment (start 138.3898 86.1988) (end 138.3898 91.7302) (width 0.2) (layer "F.Cu") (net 15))
 (segment (start 145.9621 83.7709) (end 140.8177 83.7709) (width 0.2) (layer "F.Cu") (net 15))
 (segment (start 146.87 84.6788) (end 145.9621 83.7709) (width 0.2) (layer "F.Cu") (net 15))
 (segment (start 140.8177 83.7709) (end 138.3898 86.1988) (width 0.2) (layer "F.Cu") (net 15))
 (segment (start 146.87 85.315) (end 146.87 84.6788) (width 0.2) (layer "F.Cu") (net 15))
 (segment (start 138.3898 91.7302) (end 137 93.12) (width 0.2) (layer "F.Cu") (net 15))
 (segment (start 135.8116 84.5578) (end 135.8116 94.4716) (width 0.2) (layer "F.Cu") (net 16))
 (segment (start 137.0592 83.3102) (end 135.8116 84.5578) (width 0.2) (layer "F.Cu") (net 16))
 (segment (start 147.67 85.315) (end 147.67 84.7008) (width 0.2) (layer "F.Cu") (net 16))
 (segment (start 146.2794 83.3102) (end 137.0592 83.3102) (width 0.2) (layer "F.Cu") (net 16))
 (segment (start 147.67 84.7008) (end 146.2794 83.3102) (width 0.2) (layer "F.Cu") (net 16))
 (segment (start 135.8116 94.4716) (end 137 95.66) (width 0.2) (layer "F.Cu") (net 16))
 (segment (start 157.3501 86) (end 158.5071 87.157) (width 0.2) (layer "F.Cu") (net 12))
 (segment (start 156.725 86) (end 157.3501 86) (width 0.2) (layer "F.Cu") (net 12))
 (segment (start 158.5071 87.157) (end 158.5071 88.6265) (width 0.2) (layer "F.Cu") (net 12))
 (via (at 158.5071 88.6265) (size 0.6) (drill 0.3) (layers "F.Cu" "B.Cu") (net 12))
 (segment (start 158.1049 95.0249) (end 159.04 95.96) (width 0.2) (layer "B.Cu") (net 12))
 (segment (start 158.1049 89.0287) (end 158.1049 95.0249) (width 0.2) (layer "B.Cu") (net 12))
 (segment (start 158.5071 88.6265) (end 158.1049 89.0287) (width 0.2) (layer "B.Cu") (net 12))
 (segment (start 156.725 88) (end 157.3501 88) (width 0.2) (layer "F.Cu") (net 11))
 (segment (start 157.3501 88.6222) (end 158.705 89.9771) (width 0.2) (layer "F.Cu") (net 11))
 (segment (start 157.3501 88) (end 157.3501 88.6222) (width 0.2) (layer "F.Cu") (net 11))
 (via (at 158.705 89.9771) (size 0.6) (drill 0.3) (layers "F.Cu" "B.Cu") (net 11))
 (segment (start 161.58 98.5) (end 161.58 92.8521) (width 0.2) (layer "B.Cu") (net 11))
 (segment (start 161.58 92.8521) (end 158.705 89.9771) (width 0.2) (layer "B.Cu") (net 11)))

